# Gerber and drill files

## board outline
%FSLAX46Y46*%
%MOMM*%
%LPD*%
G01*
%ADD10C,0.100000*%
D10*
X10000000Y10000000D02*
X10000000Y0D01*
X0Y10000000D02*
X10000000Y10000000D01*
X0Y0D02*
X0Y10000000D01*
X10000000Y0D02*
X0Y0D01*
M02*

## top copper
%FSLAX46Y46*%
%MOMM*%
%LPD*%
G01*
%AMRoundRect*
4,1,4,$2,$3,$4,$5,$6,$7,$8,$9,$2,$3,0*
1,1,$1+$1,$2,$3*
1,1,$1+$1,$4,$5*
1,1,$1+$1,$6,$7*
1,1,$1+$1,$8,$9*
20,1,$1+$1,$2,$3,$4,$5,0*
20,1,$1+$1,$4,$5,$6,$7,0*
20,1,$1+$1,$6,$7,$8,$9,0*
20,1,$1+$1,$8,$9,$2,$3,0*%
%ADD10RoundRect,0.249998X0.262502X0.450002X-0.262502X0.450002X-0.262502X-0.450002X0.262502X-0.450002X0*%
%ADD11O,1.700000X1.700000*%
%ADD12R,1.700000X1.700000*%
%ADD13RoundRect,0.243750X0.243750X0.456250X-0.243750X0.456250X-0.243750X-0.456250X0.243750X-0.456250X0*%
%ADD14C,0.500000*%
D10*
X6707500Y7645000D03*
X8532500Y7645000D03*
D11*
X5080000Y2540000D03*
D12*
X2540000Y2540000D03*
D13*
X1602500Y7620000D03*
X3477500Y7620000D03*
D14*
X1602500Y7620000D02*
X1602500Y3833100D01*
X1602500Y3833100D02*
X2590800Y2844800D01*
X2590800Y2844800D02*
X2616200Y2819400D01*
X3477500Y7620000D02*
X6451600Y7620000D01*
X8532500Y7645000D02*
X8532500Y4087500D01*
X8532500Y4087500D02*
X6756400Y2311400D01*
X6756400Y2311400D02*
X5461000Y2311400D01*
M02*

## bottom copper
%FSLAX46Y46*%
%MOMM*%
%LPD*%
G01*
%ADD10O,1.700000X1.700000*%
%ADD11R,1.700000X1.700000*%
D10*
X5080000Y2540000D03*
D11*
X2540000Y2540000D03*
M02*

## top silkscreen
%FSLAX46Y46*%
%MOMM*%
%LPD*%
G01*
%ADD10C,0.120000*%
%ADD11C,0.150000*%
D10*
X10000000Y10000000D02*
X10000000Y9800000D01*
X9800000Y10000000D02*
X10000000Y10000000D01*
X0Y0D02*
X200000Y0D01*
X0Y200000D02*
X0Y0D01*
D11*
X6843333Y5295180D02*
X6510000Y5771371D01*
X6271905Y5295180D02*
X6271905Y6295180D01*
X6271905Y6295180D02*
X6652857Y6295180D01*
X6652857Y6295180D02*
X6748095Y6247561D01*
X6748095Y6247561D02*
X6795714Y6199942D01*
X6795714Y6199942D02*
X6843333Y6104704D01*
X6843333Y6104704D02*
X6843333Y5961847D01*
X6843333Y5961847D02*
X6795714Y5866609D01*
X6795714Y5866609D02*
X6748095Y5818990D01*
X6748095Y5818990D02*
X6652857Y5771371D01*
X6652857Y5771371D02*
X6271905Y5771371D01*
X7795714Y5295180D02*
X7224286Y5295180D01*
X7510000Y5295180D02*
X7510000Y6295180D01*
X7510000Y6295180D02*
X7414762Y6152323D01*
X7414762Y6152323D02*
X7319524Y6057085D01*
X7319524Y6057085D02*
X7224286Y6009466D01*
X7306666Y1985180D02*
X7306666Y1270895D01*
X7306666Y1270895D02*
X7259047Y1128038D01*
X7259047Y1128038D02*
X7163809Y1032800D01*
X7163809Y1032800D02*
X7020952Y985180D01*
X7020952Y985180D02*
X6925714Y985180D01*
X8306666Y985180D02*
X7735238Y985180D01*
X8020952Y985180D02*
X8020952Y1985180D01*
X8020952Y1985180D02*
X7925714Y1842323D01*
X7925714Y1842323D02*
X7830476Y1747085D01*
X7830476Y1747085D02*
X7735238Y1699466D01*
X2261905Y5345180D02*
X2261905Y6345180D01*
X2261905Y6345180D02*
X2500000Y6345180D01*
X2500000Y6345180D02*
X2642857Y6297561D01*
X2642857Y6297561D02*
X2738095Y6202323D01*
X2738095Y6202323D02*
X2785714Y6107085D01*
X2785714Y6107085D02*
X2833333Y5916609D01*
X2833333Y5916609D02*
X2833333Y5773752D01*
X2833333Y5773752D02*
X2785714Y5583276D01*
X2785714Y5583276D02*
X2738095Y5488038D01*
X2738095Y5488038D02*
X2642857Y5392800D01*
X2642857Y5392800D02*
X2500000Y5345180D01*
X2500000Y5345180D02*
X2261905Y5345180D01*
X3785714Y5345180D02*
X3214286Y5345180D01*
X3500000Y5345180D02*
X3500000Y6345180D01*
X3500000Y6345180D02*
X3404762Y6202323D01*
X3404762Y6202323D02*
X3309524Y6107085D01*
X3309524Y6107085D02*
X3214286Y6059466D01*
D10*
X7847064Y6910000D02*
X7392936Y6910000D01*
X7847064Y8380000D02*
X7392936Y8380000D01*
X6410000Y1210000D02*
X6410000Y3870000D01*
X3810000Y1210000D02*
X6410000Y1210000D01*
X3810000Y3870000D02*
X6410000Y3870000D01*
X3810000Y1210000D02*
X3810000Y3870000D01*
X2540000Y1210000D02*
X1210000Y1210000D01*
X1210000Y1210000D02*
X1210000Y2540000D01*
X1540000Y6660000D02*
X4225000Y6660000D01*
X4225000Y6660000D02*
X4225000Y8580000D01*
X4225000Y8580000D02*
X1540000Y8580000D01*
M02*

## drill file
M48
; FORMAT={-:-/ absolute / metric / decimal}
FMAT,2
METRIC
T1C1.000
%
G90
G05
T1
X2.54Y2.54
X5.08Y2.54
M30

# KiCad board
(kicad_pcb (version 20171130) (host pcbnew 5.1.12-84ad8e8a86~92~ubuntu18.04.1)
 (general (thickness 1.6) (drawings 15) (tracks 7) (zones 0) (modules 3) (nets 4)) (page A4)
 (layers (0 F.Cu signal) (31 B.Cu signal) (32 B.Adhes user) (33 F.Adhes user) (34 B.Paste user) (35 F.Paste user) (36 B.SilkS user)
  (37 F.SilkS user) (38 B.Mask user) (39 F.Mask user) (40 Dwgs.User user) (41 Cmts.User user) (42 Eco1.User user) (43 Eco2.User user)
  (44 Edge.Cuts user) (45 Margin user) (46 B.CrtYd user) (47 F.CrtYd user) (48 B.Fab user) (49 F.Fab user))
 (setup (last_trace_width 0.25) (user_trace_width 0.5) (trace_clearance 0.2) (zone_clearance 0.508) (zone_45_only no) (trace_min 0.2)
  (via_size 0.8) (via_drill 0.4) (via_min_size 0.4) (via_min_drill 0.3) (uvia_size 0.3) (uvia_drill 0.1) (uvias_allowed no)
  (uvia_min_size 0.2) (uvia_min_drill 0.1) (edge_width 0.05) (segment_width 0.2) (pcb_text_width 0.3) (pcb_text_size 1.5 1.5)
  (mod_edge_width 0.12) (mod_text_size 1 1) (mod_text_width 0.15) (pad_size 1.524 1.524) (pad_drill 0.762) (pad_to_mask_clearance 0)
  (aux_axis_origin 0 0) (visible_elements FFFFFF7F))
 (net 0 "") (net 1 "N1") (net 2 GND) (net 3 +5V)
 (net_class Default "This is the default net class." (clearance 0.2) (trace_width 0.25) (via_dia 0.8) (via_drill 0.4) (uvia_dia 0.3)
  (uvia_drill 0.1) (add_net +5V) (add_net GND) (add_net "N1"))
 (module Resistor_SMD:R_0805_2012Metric (layer F.Cu) (at 7.62 -7.645 180)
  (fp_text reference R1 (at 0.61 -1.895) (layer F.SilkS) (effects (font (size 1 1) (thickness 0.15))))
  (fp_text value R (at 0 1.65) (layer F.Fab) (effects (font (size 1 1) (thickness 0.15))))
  (fp_line (start -0.227064 -0.735) (end 0.227064 -0.735) (layer F.SilkS) (width 0.12))
  (fp_line (start -0.227064 0.735) (end 0.227064 0.735) (layer F.SilkS) (width 0.12))
  (pad 2 smd roundrect (at 0.9125 0 180) (size 1.025 1.4) (layers F.Cu F.Paste F.Mask) (roundrect_rratio 0.2439004878048781) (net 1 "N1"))
  (pad 1 smd roundrect (at -0.9125 0 180) (size 1.025 1.4) (layers F.Cu F.Paste F.Mask) (roundrect_rratio 0.2439004878048781) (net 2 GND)))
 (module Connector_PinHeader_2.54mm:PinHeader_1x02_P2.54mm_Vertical (layer F.Cu) (at 2.54 -2.54 90)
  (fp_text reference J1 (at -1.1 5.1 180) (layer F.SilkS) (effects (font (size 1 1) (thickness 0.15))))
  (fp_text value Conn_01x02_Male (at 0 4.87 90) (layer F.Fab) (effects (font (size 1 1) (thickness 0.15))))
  (fp_line (start -1.33 3.87) (end 1.33 3.87) (layer F.SilkS) (width 0.12))
  (fp_line (start -1.33 1.27) (end -1.33 3.87) (layer F.SilkS) (width 0.12))
  (fp_line (start 1.33 1.27) (end 1.33 3.87) (layer F.SilkS) (width 0.12))
  (fp_line (start -1.33 1.27) (end 1.33 1.27) (layer F.SilkS) (width 0.12))
  (fp_line (start -1.33 0) (end -1.33 -1.33) (layer F.SilkS) (width 0.12))
  (fp_line (start -1.33 -1.33) (end 0 -1.33) (layer F.SilkS) (width 0.12))
  (pad 2 thru_hole oval (at 0 2.54 90) (size 1.7 1.7) (drill 1) (layers *.Cu *.Mask) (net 2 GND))
  (pad 1 thru_hole rect (at 0 0 90) (size 1.7 1.7) (drill 1) (layers *.Cu *.Mask) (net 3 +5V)))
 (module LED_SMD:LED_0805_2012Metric (layer F.Cu) (at 2.54 -7.62 180)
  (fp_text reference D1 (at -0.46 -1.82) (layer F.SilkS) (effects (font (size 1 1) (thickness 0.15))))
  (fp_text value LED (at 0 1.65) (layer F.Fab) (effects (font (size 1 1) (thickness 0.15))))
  (fp_line (start 1 -0.96) (end -1.685 -0.96) (layer F.SilkS) (width 0.12))
  (fp_line (start -1.685 -0.96) (end -1.685 0.96) (layer F.SilkS) (width 0.12))
  (fp_line (start -1.685 0.96) (end 1 0.96) (layer F.SilkS) (width 0.12))
  (pad 2 smd roundrect (at 0.9375 0 180) (size 0.975 1.4) (layers F.Cu F.Paste F.Mask) (roundrect_rratio 0.25) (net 3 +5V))
  (pad 1 smd roundrect (at -0.9375 0 180) (size 0.975 1.4) (layers F.Cu F.Paste F.Mask) (roundrect_rratio 0.25) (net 1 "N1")))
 (gr_line (start 10 -10) (end 10 -9.8) (layer F.SilkS) (width 0.12))
 (gr_line (start 9.8 -10) (end 10 -10) (layer F.SilkS) (width 0.12))
 (gr_line (start 0 0) (end 0.2 0) (layer F.SilkS) (width 0.12))
 (gr_line (start 0 -0.2) (end 0 0) (layer F.SilkS) (width 0.12))
 (gr_line (start 10 -10) (end 10 0) (layer Edge.Cuts) (width 0.1))
 (gr_line (start 0 -10) (end 10 -10) (layer Edge.Cuts) (width 0.1))
 (gr_line (start 0 0) (end 0 -10) (layer Edge.Cuts) (width 0.1))
 (gr_line (start 10 0) (end 0 0) (layer Edge.Cuts) (width 0.1))
 (segment (start 1.6025 -7.62) (end 1.6025 -3.8331) (width 0.5) (layer F.Cu) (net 3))
 (segment (start 1.6025 -3.8331) (end 2.5908 -2.8448) (width 0.5) (layer F.Cu) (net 3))
 (segment (start 2.5908 -2.8448) (end 2.6162 -2.8194) (width 0.5) (layer F.Cu) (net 3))
 (segment (start 3.4775 -7.62) (end 6.4516 -7.62) (width 0.5) (layer F.Cu) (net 1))
 (segment (start 8.5325 -7.645) (end 8.5325 -4.0875) (width 0.5) (layer F.Cu) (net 2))
 (segment (start 8.5325 -4.0875) (end 6.7564 -2.3114) (width 0.5) (layer F.Cu) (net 2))
 (segment (start 6.7564 -2.3114) (end 5.461 -2.3114) (width 0.5) (layer F.Cu) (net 2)))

